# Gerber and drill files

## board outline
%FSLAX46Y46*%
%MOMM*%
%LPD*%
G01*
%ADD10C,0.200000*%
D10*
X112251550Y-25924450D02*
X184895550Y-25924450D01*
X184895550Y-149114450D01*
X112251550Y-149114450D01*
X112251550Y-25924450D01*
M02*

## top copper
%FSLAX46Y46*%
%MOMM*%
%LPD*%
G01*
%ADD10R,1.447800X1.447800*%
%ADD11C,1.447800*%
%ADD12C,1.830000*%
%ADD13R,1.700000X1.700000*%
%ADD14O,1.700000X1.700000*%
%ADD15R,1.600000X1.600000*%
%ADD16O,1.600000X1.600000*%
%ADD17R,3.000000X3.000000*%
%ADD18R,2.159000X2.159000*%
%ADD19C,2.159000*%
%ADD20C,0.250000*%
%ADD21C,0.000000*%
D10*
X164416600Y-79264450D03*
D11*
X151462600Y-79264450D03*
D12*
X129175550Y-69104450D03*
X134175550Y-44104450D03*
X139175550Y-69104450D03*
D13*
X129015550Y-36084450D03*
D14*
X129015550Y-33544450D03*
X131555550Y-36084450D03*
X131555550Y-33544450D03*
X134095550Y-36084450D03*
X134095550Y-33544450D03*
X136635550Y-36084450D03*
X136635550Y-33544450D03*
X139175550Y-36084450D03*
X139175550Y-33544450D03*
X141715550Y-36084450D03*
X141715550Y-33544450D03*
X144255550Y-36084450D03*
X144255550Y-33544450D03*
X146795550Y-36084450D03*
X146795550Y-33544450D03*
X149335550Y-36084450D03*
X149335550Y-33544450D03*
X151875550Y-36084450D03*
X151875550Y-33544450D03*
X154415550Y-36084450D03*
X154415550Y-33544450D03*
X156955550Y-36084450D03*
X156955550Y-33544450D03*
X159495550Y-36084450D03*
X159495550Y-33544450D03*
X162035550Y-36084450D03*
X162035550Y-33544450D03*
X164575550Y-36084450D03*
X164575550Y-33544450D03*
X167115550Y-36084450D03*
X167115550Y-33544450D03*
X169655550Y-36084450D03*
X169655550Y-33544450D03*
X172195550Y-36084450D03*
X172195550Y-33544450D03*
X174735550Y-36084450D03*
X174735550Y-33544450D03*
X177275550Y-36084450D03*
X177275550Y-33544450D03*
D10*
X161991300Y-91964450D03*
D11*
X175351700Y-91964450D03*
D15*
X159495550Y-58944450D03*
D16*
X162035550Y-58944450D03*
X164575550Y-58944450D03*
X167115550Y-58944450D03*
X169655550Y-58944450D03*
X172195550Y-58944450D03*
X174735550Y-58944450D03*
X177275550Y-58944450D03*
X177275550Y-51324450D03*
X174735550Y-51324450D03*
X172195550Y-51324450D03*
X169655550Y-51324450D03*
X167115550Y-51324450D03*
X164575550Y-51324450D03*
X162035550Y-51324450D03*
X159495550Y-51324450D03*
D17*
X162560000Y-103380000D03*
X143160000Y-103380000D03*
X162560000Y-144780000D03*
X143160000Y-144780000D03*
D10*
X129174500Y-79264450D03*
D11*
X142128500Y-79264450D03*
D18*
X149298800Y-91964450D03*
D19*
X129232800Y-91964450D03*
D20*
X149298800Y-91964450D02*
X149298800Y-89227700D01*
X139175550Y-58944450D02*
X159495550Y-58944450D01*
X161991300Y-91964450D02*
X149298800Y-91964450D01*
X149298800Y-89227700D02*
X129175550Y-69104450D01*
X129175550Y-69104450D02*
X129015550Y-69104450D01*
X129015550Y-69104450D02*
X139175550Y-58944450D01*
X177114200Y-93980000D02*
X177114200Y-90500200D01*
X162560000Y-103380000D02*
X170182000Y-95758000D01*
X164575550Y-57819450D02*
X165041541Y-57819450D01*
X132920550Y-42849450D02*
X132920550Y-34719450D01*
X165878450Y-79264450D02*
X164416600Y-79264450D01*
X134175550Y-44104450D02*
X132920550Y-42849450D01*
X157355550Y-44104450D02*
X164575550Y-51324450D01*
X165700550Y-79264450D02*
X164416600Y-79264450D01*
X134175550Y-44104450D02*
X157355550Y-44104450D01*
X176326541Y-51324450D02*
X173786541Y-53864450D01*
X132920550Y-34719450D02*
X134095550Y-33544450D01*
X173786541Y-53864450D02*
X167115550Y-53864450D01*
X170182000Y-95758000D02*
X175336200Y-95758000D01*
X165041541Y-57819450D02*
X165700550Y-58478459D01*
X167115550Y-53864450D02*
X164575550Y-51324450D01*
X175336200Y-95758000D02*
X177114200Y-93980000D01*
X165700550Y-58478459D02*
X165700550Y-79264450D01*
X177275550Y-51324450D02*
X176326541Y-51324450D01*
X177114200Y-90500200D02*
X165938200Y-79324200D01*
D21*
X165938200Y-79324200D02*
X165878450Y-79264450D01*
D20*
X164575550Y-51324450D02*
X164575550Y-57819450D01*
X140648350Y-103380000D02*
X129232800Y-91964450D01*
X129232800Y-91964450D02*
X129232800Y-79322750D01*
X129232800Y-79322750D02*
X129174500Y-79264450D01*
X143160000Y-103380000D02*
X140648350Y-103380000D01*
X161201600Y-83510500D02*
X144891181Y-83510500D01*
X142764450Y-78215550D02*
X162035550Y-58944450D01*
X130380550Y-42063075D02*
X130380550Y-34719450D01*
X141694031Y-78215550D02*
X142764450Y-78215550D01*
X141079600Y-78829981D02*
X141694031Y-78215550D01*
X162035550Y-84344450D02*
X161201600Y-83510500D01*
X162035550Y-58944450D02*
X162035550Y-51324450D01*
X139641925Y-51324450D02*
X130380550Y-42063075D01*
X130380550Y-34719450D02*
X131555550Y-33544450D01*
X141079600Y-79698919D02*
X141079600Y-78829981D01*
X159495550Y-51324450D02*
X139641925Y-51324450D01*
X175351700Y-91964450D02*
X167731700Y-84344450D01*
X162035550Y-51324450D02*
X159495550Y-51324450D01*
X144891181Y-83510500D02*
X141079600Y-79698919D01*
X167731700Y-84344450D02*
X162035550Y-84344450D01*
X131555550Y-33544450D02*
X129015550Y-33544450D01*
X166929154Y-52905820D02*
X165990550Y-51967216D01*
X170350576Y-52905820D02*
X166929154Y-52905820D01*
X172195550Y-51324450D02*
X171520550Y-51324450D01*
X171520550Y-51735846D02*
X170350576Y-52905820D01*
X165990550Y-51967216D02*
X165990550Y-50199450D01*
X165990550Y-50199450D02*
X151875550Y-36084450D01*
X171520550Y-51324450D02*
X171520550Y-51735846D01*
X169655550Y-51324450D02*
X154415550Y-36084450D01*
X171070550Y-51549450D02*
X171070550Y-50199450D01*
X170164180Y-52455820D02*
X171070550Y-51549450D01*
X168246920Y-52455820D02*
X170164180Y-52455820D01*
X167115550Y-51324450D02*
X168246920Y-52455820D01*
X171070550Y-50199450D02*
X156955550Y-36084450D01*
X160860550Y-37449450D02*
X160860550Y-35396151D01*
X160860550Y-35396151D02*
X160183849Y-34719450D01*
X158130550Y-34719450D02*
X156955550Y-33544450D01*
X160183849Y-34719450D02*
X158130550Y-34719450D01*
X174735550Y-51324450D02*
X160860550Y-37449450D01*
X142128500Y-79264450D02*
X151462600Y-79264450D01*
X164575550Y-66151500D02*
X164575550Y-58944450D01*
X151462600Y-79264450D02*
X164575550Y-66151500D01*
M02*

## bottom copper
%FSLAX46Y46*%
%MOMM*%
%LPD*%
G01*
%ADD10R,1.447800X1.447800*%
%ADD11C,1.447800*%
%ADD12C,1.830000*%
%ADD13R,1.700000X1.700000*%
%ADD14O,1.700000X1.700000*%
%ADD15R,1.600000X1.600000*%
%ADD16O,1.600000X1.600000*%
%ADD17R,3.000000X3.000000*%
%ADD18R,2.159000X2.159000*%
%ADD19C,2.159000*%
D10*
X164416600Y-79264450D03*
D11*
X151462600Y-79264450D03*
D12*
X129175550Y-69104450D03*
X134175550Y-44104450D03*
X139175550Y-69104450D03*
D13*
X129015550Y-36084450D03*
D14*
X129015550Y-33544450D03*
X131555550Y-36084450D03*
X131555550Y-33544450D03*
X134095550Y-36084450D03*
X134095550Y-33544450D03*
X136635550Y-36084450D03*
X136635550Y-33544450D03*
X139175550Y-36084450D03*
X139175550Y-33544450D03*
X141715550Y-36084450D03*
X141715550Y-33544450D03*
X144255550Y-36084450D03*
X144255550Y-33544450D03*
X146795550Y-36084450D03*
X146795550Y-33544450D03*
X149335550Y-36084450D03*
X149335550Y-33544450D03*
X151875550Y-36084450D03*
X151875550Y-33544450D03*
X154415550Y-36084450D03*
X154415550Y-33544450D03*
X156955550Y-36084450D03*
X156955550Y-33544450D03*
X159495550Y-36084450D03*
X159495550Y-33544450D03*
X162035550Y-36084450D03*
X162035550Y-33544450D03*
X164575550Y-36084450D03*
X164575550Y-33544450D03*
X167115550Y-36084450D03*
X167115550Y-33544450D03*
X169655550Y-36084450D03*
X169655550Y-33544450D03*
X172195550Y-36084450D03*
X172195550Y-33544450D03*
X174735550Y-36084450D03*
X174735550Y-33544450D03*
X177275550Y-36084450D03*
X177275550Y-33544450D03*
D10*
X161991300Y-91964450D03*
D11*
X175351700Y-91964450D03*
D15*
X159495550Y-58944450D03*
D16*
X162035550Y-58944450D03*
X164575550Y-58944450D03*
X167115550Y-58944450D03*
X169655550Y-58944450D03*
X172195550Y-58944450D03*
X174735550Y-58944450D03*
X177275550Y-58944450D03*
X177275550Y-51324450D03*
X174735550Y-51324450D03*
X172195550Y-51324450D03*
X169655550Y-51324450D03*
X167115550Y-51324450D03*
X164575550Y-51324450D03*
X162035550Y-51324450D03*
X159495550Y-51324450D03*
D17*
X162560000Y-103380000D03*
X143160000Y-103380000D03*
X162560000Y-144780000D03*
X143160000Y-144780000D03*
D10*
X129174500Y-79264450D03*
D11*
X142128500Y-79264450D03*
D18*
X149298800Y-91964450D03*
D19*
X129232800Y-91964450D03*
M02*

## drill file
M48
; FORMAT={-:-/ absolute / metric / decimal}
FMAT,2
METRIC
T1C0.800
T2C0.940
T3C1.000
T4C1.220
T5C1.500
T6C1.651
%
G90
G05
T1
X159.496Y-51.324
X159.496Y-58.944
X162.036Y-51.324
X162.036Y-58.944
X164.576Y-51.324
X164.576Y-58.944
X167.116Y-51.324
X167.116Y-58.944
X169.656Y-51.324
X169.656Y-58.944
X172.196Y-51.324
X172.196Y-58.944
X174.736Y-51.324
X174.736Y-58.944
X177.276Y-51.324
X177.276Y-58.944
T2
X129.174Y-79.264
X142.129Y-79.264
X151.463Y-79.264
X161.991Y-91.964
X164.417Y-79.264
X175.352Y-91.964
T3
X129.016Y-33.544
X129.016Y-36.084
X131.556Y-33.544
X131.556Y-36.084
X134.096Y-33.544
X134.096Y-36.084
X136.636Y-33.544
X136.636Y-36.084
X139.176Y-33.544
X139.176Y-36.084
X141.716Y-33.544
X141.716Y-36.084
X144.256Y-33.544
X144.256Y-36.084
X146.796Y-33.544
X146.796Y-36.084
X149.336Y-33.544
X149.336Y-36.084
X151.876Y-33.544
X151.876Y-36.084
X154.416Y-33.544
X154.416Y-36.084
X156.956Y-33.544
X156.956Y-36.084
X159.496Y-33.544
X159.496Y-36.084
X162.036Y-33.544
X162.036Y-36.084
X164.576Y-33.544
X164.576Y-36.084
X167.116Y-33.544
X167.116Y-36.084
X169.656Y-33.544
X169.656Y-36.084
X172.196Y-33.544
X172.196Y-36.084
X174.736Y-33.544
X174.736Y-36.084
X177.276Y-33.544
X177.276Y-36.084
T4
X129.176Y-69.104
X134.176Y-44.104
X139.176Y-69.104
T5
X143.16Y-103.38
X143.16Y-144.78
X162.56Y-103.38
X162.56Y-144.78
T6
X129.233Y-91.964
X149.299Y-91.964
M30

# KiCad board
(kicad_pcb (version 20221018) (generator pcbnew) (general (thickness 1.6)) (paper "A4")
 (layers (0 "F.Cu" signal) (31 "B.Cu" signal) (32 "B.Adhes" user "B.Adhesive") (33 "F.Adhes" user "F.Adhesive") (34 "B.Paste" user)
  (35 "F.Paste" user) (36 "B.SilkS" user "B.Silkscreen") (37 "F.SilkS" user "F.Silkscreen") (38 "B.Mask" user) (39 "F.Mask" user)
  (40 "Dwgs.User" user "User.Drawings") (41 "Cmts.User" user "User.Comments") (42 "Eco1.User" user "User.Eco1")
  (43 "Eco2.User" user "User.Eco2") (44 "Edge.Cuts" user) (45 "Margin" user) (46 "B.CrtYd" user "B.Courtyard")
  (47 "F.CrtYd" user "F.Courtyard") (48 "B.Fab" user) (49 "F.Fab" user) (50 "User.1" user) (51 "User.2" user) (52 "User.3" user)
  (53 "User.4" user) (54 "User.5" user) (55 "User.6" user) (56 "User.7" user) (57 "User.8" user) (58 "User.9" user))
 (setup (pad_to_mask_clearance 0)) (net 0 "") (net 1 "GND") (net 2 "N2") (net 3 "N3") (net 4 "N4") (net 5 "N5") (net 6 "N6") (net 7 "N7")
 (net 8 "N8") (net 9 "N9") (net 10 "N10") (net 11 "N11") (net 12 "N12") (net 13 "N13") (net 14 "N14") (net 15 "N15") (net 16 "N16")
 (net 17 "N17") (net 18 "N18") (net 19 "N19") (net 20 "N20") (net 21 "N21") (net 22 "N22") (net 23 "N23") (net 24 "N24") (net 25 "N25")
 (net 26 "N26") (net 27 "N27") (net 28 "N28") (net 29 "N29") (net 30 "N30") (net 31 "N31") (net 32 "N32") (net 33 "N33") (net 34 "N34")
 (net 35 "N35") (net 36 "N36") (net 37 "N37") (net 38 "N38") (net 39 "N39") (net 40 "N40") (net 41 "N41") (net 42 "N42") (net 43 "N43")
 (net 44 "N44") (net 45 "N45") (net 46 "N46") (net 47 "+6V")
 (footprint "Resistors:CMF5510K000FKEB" (layer "F.Cu") (at 164.4166 79.26445 180)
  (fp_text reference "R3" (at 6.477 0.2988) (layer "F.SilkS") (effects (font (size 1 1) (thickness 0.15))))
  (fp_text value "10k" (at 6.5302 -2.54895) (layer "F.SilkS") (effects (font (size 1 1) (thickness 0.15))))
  (pad "1" thru_hole rect (at 0 0 180) (size 1.4478 1.4478) (drill 0.9398) (layers "*.Cu" "*.Mask") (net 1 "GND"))
  (pad "2" thru_hole circle (at 12.954 0 180) (size 1.4478 1.4478) (drill 0.9398) (layers "*.Cu" "*.Mask") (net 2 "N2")))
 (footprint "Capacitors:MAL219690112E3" (layer "F.Cu") (at 129.17555 69.10445)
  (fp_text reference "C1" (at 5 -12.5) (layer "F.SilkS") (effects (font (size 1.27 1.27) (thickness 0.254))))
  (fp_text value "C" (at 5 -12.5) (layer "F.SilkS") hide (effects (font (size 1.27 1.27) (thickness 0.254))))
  (pad "1" thru_hole circle (at 0 0) (size 1.83 1.83) (drill 1.22) (layers "*.Cu" "*.Mask") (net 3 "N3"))
  (pad "2" thru_hole circle (at 5 -25) (size 1.83 1.83) (drill 1.22) (layers "*.Cu" "*.Mask") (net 1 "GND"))
  (pad "3" thru_hole circle (at 10 0) (size 1.83 1.83) (drill 1.22) (layers "*.Cu" "*.Mask")))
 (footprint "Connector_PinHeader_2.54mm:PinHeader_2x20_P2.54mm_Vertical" (layer "F.Cu") (at 129.01555 36.08445 90)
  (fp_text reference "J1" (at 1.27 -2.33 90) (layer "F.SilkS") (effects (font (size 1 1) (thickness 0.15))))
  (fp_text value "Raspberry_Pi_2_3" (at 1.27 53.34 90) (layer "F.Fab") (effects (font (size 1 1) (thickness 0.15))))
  (pad "1" thru_hole rect (at 0 0 90) (size 1.7 1.7) (drill 1) (layers "*.Cu" "*.Mask") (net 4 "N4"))
  (pad "2" thru_hole oval (at 2.54 0 90) (size 1.7 1.7) (drill 1) (layers "*.Cu" "*.Mask") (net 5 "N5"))
  (pad "3" thru_hole oval (at 0 2.54 90) (size 1.7 1.7) (drill 1) (layers "*.Cu" "*.Mask") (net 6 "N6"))
  (pad "4" thru_hole oval (at 2.54 2.54 90) (size 1.7 1.7) (drill 1) (layers "*.Cu" "*.Mask") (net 5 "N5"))
  (pad "5" thru_hole oval (at 0 5.08 90) (size 1.7 1.7) (drill 1) (layers "*.Cu" "*.Mask") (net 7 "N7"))
  (pad "6" thru_hole oval (at 2.54 5.08 90) (size 1.7 1.7) (drill 1) (layers "*.Cu" "*.Mask") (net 1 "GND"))
  (pad "7" thru_hole oval (at 0 7.62 90) (size 1.7 1.7) (drill 1) (layers "*.Cu" "*.Mask") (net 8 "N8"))
  (pad "8" thru_hole oval (at 2.54 7.62 90) (size 1.7 1.7) (drill 1) (layers "*.Cu" "*.Mask") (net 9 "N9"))
  (pad "9" thru_hole oval (at 0 10.16 90) (size 1.7 1.7) (drill 1) (layers "*.Cu" "*.Mask") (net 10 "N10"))
  (pad "10" thru_hole oval (at 2.54 10.16 90) (size 1.7 1.7) (drill 1) (layers "*.Cu" "*.Mask") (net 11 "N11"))
  (pad "11" thru_hole oval (at 0 12.7 90) (size 1.7 1.7) (drill 1) (layers "*.Cu" "*.Mask") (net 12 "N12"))
  (pad "12" thru_hole oval (at 2.54 12.7 90) (size 1.7 1.7) (drill 1) (layers "*.Cu" "*.Mask") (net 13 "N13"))
  (pad "13" thru_hole oval (at 0 15.24 90) (size 1.7 1.7) (drill 1) (layers "*.Cu" "*.Mask") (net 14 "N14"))
  (pad "14" thru_hole oval (at 2.54 15.24 90) (size 1.7 1.7) (drill 1) (layers "*.Cu" "*.Mask") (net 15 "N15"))
  (pad "15" thru_hole oval (at 0 17.78 90) (size 1.7 1.7) (drill 1) (layers "*.Cu" "*.Mask") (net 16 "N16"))
  (pad "16" thru_hole oval (at 2.54 17.78 90) (size 1.7 1.7) (drill 1) (layers "*.Cu" "*.Mask") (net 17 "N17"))
  (pad "17" thru_hole oval (at 0 20.32 90) (size 1.7 1.7) (drill 1) (layers "*.Cu" "*.Mask") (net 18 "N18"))
  (pad "18" thru_hole oval (at 2.54 20.32 90) (size 1.7 1.7) (drill 1) (layers "*.Cu" "*.Mask") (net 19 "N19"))
  (pad "19" thru_hole oval (at 0 22.86 90) (size 1.7 1.7) (drill 1) (layers "*.Cu" "*.Mask") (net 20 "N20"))
  (pad "20" thru_hole oval (at 2.54 22.86 90) (size 1.7 1.7) (drill 1) (layers "*.Cu" "*.Mask") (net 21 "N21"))
  (pad "21" thru_hole oval (at 0 25.4 90) (size 1.7 1.7) (drill 1) (layers "*.Cu" "*.Mask") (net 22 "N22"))
  (pad "22" thru_hole oval (at 2.54 25.4 90) (size 1.7 1.7) (drill 1) (layers "*.Cu" "*.Mask") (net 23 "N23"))
  (pad "23" thru_hole oval (at 0 27.94 90) (size 1.7 1.7) (drill 1) (layers "*.Cu" "*.Mask") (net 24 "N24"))
  (pad "24" thru_hole oval (at 2.54 27.94 90) (size 1.7 1.7) (drill 1) (layers "*.Cu" "*.Mask") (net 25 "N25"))
  (pad "25" thru_hole oval (at 0 30.48 90) (size 1.7 1.7) (drill 1) (layers "*.Cu" "*.Mask") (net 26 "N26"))
  (pad "26" thru_hole oval (at 2.54 30.48 90) (size 1.7 1.7) (drill 1) (layers "*.Cu" "*.Mask") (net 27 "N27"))
  (pad "27" thru_hole oval (at 0 33.02 90) (size 1.7 1.7) (drill 1) (layers "*.Cu" "*.Mask") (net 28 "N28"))
  (pad "28" thru_hole oval (at 2.54 33.02 90) (size 1.7 1.7) (drill 1) (layers "*.Cu" "*.Mask") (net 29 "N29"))
  (pad "29" thru_hole oval (at 0 35.56 90) (size 1.7 1.7) (drill 1) (layers "*.Cu" "*.Mask") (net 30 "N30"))
  (pad "30" thru_hole oval (at 2.54 35.56 90) (size 1.7 1.7) (drill 1) (layers "*.Cu" "*.Mask") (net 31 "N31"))
  (pad "31" thru_hole oval (at 0 38.1 90) (size 1.7 1.7) (drill 1) (layers "*.Cu" "*.Mask") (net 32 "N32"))
  (pad "32" thru_hole oval (at 2.54 38.1 90) (size 1.7 1.7) (drill 1) (layers "*.Cu" "*.Mask") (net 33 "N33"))
  (pad "33" thru_hole oval (at 0 40.64 90) (size 1.7 1.7) (drill 1) (layers "*.Cu" "*.Mask") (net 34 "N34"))
  (pad "34" thru_hole oval (at 2.54 40.64 90) (size 1.7 1.7) (drill 1) (layers "*.Cu" "*.Mask") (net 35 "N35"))
  (pad "35" thru_hole oval (at 0 43.18 90) (size 1.7 1.7) (drill 1) (layers "*.Cu" "*.Mask") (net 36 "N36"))
  (pad "36" thru_hole oval (at 2.54 43.18 90) (size 1.7 1.7) (drill 1) (layers "*.Cu" "*.Mask") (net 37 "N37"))
  (pad "37" thru_hole oval (at 0 45.72 90) (size 1.7 1.7) (drill 1) (layers "*.Cu" "*.Mask") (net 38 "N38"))
  (pad "38" thru_hole oval (at 2.54 45.72 90) (size 1.7 1.7) (drill 1) (layers "*.Cu" "*.Mask") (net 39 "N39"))
  (pad "39" thru_hole oval (at 0 48.26 90) (size 1.7 1.7) (drill 1) (layers "*.Cu" "*.Mask") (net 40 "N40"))
  (pad "40" thru_hole oval (at 2.54 48.26 90) (size 1.7 1.7) (drill 1) (layers "*.Cu" "*.Mask") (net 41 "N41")))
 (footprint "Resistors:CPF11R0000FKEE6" (layer "F.Cu") (at 161.9913 91.96445)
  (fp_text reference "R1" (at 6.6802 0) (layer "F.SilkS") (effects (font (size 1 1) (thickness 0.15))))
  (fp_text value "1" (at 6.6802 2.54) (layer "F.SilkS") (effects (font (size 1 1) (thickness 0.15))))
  (pad "1" thru_hole rect (at 0 0) (size 1.4478 1.4478) (drill 0.9398) (layers "*.Cu" "*.Mask") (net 3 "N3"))
  (pad "2" thru_hole circle (at 13.3604 0) (size 1.4478 1.4478) (drill 0.9398) (layers "*.Cu" "*.Mask") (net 5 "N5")))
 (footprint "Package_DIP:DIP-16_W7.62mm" (layer "F.Cu") (at 159.49555 58.94445 90)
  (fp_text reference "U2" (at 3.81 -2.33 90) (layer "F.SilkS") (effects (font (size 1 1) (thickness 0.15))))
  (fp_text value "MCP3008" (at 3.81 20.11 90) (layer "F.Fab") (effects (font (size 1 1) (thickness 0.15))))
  (pad "1" thru_hole rect (at 0 0 90) (size 1.6 1.6) (drill 0.8) (layers "*.Cu" "*.Mask") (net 3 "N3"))
  (pad "2" thru_hole oval (at 0 2.54 90) (size 1.6 1.6) (drill 0.8) (layers "*.Cu" "*.Mask") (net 5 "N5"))
  (pad "3" thru_hole oval (at 0 5.08 90) (size 1.6 1.6) (drill 0.8) (layers "*.Cu" "*.Mask") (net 2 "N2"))
  (pad "4" thru_hole oval (at 0 7.62 90) (size 1.6 1.6) (drill 0.8) (layers "*.Cu" "*.Mask") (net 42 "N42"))
  (pad "5" thru_hole oval (at 0 10.16 90) (size 1.6 1.6) (drill 0.8) (layers "*.Cu" "*.Mask") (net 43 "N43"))
  (pad "6" thru_hole oval (at 0 12.7 90) (size 1.6 1.6) (drill 0.8) (layers "*.Cu" "*.Mask") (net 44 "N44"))
  (pad "7" thru_hole oval (at 0 15.24 90) (size 1.6 1.6) (drill 0.8) (layers "*.Cu" "*.Mask") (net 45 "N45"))
  (pad "8" thru_hole oval (at 0 17.78 90) (size 1.6 1.6) (drill 0.8) (layers "*.Cu" "*.Mask") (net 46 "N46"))
  (pad "9" thru_hole oval (at 7.62 17.78 90) (size 1.6 1.6) (drill 0.8) (layers "*.Cu" "*.Mask") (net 1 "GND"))
  (pad "10" thru_hole oval (at 7.62 15.24 90) (size 1.6 1.6) (drill 0.8) (layers "*.Cu" "*.Mask") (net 25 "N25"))
  (pad "11" thru_hole oval (at 7.62 12.7 90) (size 1.6 1.6) (drill 0.8) (layers "*.Cu" "*.Mask") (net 20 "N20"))
  (pad "12" thru_hole oval (at 7.62 10.16 90) (size 1.6 1.6) (drill 0.8) (layers "*.Cu" "*.Mask") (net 22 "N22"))
  (pad "13" thru_hole oval (at 7.62 7.62 90) (size 1.6 1.6) (drill 0.8) (layers "*.Cu" "*.Mask") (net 24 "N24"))
  (pad "14" thru_hole oval (at 7.62 5.08 90) (size 1.6 1.6) (drill 0.8) (layers "*.Cu" "*.Mask") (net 1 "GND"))
  (pad "15" thru_hole oval (at 7.62 2.54 90) (size 1.6 1.6) (drill 0.8) (layers "*.Cu" "*.Mask") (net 5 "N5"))
  (pad "16" thru_hole oval (at 7.62 0 90) (size 1.6 1.6) (drill 0.8) (layers "*.Cu" "*.Mask") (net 5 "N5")))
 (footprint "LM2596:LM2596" (layer "F.Cu") (at 152.4 124.46 -90)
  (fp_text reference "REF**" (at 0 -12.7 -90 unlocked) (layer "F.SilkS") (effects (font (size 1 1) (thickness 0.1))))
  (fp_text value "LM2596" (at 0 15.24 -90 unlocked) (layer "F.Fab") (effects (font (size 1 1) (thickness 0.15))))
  (pad "1" thru_hole rect (at -21.08 -10.16 270) (size 3 3) (drill 1.5) (layers "*.Cu" "*.Mask") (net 1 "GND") (thermal_bridge_angle 45))
  (pad "2" thru_hole rect (at -21.08 9.24 270) (size 3 3) (drill 1.5) (layers "*.Cu" "*.Mask") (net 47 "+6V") (thermal_bridge_angle 45))
  (pad "3" thru_hole rect (at 20.32 -10.16 270) (size 3 3) (drill 1.5) (layers "*.Cu" "*.Mask") (thermal_bridge_angle 45))
  (pad "4" thru_hole rect (at 20.32 9.24 270) (size 3 3) (drill 1.5) (layers "*.Cu" "*.Mask") (thermal_bridge_angle 45)))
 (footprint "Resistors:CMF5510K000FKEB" (layer "F.Cu") (at 129.1745 79.26445)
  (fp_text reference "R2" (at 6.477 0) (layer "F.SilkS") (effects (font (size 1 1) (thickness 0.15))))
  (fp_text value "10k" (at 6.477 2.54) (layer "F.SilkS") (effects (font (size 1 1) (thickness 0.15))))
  (pad "1" thru_hole rect (at 0 0) (size 1.4478 1.4478) (drill 0.9398) (layers "*.Cu" "*.Mask") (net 47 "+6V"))
  (pad "2" thru_hole circle (at 12.954 0) (size 1.4478 1.4478) (drill 0.9398) (layers "*.Cu" "*.Mask") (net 2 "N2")))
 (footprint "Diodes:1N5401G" (layer "F.Cu") (at 149.2988 91.96445 180)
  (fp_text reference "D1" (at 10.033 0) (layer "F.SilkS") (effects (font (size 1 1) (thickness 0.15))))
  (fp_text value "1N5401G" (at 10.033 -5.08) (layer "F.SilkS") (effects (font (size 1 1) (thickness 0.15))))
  (pad "1" thru_hole rect (at 0 0 180) (size 2.159 2.159) (drill 1.651) (layers "*.Cu" "*.Mask") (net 3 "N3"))
  (pad "2" thru_hole circle (at 20.066 0 180) (size 2.159 2.159) (drill 1.651) (layers "*.Cu" "*.Mask") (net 47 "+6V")))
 (gr_rect (start 112.25155 25.92445) (end 184.89555 149.11445) (stroke (width 0.2) (type default)) (fill none) (layer "Edge.Cuts"))
 (segment (start 149.2988 91.96445) (end 149.2988 89.2277) (width 0.25) (layer "F.Cu") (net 3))
 (segment (start 139.17555 58.94445) (end 159.49555 58.94445) (width 0.25) (layer "F.Cu") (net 3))
 (segment (start 161.9913 91.96445) (end 149.2988 91.96445) (width 0.25) (layer "F.Cu") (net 3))
 (segment (start 149.2988 89.2277) (end 129.17555 69.10445) (width 0.25) (layer "F.Cu") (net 3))
 (segment (start 129.17555 69.10445) (end 129.01555 69.10445) (width 0.25) (layer "F.Cu") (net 3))
 (segment (start 129.01555 69.10445) (end 139.17555 58.94445) (width 0.25) (layer "F.Cu") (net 3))
 (segment (start 177.1142 93.98) (end 177.1142 90.5002) (width 0.25) (layer "F.Cu") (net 1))
 (segment (start 162.56 103.38) (end 170.182 95.758) (width 0.25) (layer "F.Cu") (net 1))
 (segment (start 164.57555 57.81945) (end 165.041541 57.81945) (width 0.25) (layer "F.Cu") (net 1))
 (segment (start 132.92055 42.84945) (end 132.92055 34.71945) (width 0.25) (layer "F.Cu") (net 1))
 (segment (start 165.87845 79.26445) (end 164.4166 79.26445) (width 0.25) (layer "F.Cu") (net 1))
 (segment (start 134.17555 44.10445) (end 132.92055 42.84945) (width 0.25) (layer "F.Cu") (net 1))
 (segment (start 157.35555 44.10445) (end 164.57555 51.32445) (width 0.25) (layer "F.Cu") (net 1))
 (segment (start 165.70055 79.26445) (end 164.4166 79.26445) (width 0.25) (layer "F.Cu") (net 1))
 (segment (start 134.17555 44.10445) (end 157.35555 44.10445) (width 0.25) (layer "F.Cu") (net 1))
 (segment (start 176.326541 51.32445) (end 173.786541 53.86445) (width 0.25) (layer "F.Cu") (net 1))
 (segment (start 132.92055 34.71945) (end 134.09555 33.54445) (width 0.25) (layer "F.Cu") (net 1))
 (segment (start 173.786541 53.86445) (end 167.11555 53.86445) (width 0.25) (layer "F.Cu") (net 1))
 (segment (start 170.182 95.758) (end 175.3362 95.758) (width 0.25) (layer "F.Cu") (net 1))
 (segment (start 165.041541 57.81945) (end 165.70055 58.478459) (width 0.25) (layer "F.Cu") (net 1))
 (segment (start 167.11555 53.86445) (end 164.57555 51.32445) (width 0.25) (layer "F.Cu") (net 1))
 (segment (start 175.3362 95.758) (end 177.1142 93.98) (width 0.25) (layer "F.Cu") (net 1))
 (segment (start 165.70055 58.478459) (end 165.70055 79.26445) (width 0.25) (layer "F.Cu") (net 1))
 (segment (start 177.27555 51.32445) (end 176.326541 51.32445) (width 0.25) (layer "F.Cu") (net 1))
 (segment (start 177.1142 90.5002) (end 165.9382 79.3242) (width 0.25) (layer "F.Cu") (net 1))
 (segment (start 165.9382 79.3242) (end 165.87845 79.26445) (width 0) (layer "F.Cu") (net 1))
 (segment (start 164.57555 51.32445) (end 164.57555 57.81945) (width 0.25) (layer "F.Cu") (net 1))
 (segment (start 140.64835 103.38) (end 129.2328 91.96445) (width 0.25) (layer "F.Cu") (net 47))
 (segment (start 129.2328 91.96445) (end 129.2328 79.32275) (width 0.25) (layer "F.Cu") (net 47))
 (segment (start 129.2328 79.32275) (end 129.1745 79.26445) (width 0.25) (layer "F.Cu") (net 47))
 (segment (start 143.16 103.38) (end 140.64835 103.38) (width 0.25) (layer "F.Cu") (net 47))
 (segment (start 161.2016 83.5105) (end 144.891181 83.5105) (width 0.25) (layer "F.Cu") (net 5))
 (segment (start 142.76445 78.21555) (end 162.03555 58.94445) (width 0.25) (layer "F.Cu") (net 5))
 (segment (start 130.38055 42.063075) (end 130.38055 34.71945) (width 0.25) (layer "F.Cu") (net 5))
 (segment (start 141.694031 78.21555) (end 142.76445 78.21555) (width 0.25) (layer "F.Cu") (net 5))
 (segment (start 141.0796 78.829981) (end 141.694031 78.21555) (width 0.25) (layer "F.Cu") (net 5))
 (segment (start 162.03555 84.34445) (end 161.2016 83.5105) (width 0.25) (layer "F.Cu") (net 5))
 (segment (start 162.03555 58.94445) (end 162.03555 51.32445) (width 0.25) (layer "F.Cu") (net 5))
 (segment (start 139.641925 51.32445) (end 130.38055 42.063075) (width 0.25) (layer "F.Cu") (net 5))
 (segment (start 130.38055 34.71945) (end 131.55555 33.54445) (width 0.25) (layer "F.Cu") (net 5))
 (segment (start 141.0796 79.698919) (end 141.0796 78.829981) (width 0.25) (layer "F.Cu") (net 5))
 (segment (start 159.49555 51.32445) (end 139.641925 51.32445) (width 0.25) (layer "F.Cu") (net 5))
 (segment (start 175.3517 91.96445) (end 167.7317 84.34445) (width 0.25) (layer "F.Cu") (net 5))
 (segment (start 162.03555 51.32445) (end 159.49555 51.32445) (width 0.25) (layer "F.Cu") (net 5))
 (segment (start 144.891181 83.5105) (end 141.0796 79.698919) (width 0.25) (layer "F.Cu") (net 5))
 (segment (start 167.7317 84.34445) (end 162.03555 84.34445) (width 0.25) (layer "F.Cu") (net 5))
 (segment (start 131.55555 33.54445) (end 129.01555 33.54445) (width 0.25) (layer "F.Cu") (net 5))
 (segment (start 166.929154 52.90582) (end 165.99055 51.967216) (width 0.25) (layer "F.Cu") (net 20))
 (segment (start 170.350576 52.90582) (end 166.929154 52.90582) (width 0.25) (layer "F.Cu") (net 20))
 (segment (start 172.19555 51.32445) (end 171.52055 51.32445) (width 0.25) (layer "F.Cu") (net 20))
 (segment (start 171.52055 51.735846) (end 170.350576 52.90582) (width 0.25) (layer "F.Cu") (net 20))
 (segment (start 165.99055 51.967216) (end 165.99055 50.19945) (width 0.25) (layer "F.Cu") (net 20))
 (segment (start 165.99055 50.19945) (end 151.87555 36.08445) (width 0.25) (layer "F.Cu") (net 20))
 (segment (start 171.52055 51.32445) (end 171.52055 51.735846) (width 0.25) (layer "F.Cu") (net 20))
 (segment (start 169.65555 51.32445) (end 154.41555 36.08445) (width 0.25) (layer "F.Cu") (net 22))
 (segment (start 171.07055 51.54945) (end 171.07055 50.19945) (width 0.25) (layer "F.Cu") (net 24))
 (segment (start 170.16418 52.45582) (end 171.07055 51.54945) (width 0.25) (layer "F.Cu") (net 24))
 (segment (start 168.24692 52.45582) (end 170.16418 52.45582) (width 0.25) (layer "F.Cu") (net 24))
 (segment (start 167.11555 51.32445) (end 168.24692 52.45582) (width 0.25) (layer "F.Cu") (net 24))
 (segment (start 171.07055 50.19945) (end 156.95555 36.08445) (width 0.25) (layer "F.Cu") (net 24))
 (segment (start 160.86055 37.44945) (end 160.86055 35.396151) (width 0.25) (layer "F.Cu") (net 25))
 (segment (start 160.86055 35.396151) (end 160.183849 34.71945) (width 0.25) (layer "F.Cu") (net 25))
 (segment (start 158.13055 34.71945) (end 156.95555 33.54445) (width 0.25) (layer "F.Cu") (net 25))
 (segment (start 160.183849 34.71945) (end 158.13055 34.71945) (width 0.25) (layer "F.Cu") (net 25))
 (segment (start 174.73555 51.32445) (end 160.86055 37.44945) (width 0.25) (layer "F.Cu") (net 25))
 (segment (start 142.1285 79.26445) (end 151.4626 79.26445) (width 0.25) (layer "F.Cu") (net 2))
 (segment (start 164.57555 66.1515) (end 164.57555 58.94445) (width 0.25) (layer "F.Cu") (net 2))
 (segment (start 151.4626 79.26445) (end 164.57555 66.1515) (width 0.25) (layer "F.Cu") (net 2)))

